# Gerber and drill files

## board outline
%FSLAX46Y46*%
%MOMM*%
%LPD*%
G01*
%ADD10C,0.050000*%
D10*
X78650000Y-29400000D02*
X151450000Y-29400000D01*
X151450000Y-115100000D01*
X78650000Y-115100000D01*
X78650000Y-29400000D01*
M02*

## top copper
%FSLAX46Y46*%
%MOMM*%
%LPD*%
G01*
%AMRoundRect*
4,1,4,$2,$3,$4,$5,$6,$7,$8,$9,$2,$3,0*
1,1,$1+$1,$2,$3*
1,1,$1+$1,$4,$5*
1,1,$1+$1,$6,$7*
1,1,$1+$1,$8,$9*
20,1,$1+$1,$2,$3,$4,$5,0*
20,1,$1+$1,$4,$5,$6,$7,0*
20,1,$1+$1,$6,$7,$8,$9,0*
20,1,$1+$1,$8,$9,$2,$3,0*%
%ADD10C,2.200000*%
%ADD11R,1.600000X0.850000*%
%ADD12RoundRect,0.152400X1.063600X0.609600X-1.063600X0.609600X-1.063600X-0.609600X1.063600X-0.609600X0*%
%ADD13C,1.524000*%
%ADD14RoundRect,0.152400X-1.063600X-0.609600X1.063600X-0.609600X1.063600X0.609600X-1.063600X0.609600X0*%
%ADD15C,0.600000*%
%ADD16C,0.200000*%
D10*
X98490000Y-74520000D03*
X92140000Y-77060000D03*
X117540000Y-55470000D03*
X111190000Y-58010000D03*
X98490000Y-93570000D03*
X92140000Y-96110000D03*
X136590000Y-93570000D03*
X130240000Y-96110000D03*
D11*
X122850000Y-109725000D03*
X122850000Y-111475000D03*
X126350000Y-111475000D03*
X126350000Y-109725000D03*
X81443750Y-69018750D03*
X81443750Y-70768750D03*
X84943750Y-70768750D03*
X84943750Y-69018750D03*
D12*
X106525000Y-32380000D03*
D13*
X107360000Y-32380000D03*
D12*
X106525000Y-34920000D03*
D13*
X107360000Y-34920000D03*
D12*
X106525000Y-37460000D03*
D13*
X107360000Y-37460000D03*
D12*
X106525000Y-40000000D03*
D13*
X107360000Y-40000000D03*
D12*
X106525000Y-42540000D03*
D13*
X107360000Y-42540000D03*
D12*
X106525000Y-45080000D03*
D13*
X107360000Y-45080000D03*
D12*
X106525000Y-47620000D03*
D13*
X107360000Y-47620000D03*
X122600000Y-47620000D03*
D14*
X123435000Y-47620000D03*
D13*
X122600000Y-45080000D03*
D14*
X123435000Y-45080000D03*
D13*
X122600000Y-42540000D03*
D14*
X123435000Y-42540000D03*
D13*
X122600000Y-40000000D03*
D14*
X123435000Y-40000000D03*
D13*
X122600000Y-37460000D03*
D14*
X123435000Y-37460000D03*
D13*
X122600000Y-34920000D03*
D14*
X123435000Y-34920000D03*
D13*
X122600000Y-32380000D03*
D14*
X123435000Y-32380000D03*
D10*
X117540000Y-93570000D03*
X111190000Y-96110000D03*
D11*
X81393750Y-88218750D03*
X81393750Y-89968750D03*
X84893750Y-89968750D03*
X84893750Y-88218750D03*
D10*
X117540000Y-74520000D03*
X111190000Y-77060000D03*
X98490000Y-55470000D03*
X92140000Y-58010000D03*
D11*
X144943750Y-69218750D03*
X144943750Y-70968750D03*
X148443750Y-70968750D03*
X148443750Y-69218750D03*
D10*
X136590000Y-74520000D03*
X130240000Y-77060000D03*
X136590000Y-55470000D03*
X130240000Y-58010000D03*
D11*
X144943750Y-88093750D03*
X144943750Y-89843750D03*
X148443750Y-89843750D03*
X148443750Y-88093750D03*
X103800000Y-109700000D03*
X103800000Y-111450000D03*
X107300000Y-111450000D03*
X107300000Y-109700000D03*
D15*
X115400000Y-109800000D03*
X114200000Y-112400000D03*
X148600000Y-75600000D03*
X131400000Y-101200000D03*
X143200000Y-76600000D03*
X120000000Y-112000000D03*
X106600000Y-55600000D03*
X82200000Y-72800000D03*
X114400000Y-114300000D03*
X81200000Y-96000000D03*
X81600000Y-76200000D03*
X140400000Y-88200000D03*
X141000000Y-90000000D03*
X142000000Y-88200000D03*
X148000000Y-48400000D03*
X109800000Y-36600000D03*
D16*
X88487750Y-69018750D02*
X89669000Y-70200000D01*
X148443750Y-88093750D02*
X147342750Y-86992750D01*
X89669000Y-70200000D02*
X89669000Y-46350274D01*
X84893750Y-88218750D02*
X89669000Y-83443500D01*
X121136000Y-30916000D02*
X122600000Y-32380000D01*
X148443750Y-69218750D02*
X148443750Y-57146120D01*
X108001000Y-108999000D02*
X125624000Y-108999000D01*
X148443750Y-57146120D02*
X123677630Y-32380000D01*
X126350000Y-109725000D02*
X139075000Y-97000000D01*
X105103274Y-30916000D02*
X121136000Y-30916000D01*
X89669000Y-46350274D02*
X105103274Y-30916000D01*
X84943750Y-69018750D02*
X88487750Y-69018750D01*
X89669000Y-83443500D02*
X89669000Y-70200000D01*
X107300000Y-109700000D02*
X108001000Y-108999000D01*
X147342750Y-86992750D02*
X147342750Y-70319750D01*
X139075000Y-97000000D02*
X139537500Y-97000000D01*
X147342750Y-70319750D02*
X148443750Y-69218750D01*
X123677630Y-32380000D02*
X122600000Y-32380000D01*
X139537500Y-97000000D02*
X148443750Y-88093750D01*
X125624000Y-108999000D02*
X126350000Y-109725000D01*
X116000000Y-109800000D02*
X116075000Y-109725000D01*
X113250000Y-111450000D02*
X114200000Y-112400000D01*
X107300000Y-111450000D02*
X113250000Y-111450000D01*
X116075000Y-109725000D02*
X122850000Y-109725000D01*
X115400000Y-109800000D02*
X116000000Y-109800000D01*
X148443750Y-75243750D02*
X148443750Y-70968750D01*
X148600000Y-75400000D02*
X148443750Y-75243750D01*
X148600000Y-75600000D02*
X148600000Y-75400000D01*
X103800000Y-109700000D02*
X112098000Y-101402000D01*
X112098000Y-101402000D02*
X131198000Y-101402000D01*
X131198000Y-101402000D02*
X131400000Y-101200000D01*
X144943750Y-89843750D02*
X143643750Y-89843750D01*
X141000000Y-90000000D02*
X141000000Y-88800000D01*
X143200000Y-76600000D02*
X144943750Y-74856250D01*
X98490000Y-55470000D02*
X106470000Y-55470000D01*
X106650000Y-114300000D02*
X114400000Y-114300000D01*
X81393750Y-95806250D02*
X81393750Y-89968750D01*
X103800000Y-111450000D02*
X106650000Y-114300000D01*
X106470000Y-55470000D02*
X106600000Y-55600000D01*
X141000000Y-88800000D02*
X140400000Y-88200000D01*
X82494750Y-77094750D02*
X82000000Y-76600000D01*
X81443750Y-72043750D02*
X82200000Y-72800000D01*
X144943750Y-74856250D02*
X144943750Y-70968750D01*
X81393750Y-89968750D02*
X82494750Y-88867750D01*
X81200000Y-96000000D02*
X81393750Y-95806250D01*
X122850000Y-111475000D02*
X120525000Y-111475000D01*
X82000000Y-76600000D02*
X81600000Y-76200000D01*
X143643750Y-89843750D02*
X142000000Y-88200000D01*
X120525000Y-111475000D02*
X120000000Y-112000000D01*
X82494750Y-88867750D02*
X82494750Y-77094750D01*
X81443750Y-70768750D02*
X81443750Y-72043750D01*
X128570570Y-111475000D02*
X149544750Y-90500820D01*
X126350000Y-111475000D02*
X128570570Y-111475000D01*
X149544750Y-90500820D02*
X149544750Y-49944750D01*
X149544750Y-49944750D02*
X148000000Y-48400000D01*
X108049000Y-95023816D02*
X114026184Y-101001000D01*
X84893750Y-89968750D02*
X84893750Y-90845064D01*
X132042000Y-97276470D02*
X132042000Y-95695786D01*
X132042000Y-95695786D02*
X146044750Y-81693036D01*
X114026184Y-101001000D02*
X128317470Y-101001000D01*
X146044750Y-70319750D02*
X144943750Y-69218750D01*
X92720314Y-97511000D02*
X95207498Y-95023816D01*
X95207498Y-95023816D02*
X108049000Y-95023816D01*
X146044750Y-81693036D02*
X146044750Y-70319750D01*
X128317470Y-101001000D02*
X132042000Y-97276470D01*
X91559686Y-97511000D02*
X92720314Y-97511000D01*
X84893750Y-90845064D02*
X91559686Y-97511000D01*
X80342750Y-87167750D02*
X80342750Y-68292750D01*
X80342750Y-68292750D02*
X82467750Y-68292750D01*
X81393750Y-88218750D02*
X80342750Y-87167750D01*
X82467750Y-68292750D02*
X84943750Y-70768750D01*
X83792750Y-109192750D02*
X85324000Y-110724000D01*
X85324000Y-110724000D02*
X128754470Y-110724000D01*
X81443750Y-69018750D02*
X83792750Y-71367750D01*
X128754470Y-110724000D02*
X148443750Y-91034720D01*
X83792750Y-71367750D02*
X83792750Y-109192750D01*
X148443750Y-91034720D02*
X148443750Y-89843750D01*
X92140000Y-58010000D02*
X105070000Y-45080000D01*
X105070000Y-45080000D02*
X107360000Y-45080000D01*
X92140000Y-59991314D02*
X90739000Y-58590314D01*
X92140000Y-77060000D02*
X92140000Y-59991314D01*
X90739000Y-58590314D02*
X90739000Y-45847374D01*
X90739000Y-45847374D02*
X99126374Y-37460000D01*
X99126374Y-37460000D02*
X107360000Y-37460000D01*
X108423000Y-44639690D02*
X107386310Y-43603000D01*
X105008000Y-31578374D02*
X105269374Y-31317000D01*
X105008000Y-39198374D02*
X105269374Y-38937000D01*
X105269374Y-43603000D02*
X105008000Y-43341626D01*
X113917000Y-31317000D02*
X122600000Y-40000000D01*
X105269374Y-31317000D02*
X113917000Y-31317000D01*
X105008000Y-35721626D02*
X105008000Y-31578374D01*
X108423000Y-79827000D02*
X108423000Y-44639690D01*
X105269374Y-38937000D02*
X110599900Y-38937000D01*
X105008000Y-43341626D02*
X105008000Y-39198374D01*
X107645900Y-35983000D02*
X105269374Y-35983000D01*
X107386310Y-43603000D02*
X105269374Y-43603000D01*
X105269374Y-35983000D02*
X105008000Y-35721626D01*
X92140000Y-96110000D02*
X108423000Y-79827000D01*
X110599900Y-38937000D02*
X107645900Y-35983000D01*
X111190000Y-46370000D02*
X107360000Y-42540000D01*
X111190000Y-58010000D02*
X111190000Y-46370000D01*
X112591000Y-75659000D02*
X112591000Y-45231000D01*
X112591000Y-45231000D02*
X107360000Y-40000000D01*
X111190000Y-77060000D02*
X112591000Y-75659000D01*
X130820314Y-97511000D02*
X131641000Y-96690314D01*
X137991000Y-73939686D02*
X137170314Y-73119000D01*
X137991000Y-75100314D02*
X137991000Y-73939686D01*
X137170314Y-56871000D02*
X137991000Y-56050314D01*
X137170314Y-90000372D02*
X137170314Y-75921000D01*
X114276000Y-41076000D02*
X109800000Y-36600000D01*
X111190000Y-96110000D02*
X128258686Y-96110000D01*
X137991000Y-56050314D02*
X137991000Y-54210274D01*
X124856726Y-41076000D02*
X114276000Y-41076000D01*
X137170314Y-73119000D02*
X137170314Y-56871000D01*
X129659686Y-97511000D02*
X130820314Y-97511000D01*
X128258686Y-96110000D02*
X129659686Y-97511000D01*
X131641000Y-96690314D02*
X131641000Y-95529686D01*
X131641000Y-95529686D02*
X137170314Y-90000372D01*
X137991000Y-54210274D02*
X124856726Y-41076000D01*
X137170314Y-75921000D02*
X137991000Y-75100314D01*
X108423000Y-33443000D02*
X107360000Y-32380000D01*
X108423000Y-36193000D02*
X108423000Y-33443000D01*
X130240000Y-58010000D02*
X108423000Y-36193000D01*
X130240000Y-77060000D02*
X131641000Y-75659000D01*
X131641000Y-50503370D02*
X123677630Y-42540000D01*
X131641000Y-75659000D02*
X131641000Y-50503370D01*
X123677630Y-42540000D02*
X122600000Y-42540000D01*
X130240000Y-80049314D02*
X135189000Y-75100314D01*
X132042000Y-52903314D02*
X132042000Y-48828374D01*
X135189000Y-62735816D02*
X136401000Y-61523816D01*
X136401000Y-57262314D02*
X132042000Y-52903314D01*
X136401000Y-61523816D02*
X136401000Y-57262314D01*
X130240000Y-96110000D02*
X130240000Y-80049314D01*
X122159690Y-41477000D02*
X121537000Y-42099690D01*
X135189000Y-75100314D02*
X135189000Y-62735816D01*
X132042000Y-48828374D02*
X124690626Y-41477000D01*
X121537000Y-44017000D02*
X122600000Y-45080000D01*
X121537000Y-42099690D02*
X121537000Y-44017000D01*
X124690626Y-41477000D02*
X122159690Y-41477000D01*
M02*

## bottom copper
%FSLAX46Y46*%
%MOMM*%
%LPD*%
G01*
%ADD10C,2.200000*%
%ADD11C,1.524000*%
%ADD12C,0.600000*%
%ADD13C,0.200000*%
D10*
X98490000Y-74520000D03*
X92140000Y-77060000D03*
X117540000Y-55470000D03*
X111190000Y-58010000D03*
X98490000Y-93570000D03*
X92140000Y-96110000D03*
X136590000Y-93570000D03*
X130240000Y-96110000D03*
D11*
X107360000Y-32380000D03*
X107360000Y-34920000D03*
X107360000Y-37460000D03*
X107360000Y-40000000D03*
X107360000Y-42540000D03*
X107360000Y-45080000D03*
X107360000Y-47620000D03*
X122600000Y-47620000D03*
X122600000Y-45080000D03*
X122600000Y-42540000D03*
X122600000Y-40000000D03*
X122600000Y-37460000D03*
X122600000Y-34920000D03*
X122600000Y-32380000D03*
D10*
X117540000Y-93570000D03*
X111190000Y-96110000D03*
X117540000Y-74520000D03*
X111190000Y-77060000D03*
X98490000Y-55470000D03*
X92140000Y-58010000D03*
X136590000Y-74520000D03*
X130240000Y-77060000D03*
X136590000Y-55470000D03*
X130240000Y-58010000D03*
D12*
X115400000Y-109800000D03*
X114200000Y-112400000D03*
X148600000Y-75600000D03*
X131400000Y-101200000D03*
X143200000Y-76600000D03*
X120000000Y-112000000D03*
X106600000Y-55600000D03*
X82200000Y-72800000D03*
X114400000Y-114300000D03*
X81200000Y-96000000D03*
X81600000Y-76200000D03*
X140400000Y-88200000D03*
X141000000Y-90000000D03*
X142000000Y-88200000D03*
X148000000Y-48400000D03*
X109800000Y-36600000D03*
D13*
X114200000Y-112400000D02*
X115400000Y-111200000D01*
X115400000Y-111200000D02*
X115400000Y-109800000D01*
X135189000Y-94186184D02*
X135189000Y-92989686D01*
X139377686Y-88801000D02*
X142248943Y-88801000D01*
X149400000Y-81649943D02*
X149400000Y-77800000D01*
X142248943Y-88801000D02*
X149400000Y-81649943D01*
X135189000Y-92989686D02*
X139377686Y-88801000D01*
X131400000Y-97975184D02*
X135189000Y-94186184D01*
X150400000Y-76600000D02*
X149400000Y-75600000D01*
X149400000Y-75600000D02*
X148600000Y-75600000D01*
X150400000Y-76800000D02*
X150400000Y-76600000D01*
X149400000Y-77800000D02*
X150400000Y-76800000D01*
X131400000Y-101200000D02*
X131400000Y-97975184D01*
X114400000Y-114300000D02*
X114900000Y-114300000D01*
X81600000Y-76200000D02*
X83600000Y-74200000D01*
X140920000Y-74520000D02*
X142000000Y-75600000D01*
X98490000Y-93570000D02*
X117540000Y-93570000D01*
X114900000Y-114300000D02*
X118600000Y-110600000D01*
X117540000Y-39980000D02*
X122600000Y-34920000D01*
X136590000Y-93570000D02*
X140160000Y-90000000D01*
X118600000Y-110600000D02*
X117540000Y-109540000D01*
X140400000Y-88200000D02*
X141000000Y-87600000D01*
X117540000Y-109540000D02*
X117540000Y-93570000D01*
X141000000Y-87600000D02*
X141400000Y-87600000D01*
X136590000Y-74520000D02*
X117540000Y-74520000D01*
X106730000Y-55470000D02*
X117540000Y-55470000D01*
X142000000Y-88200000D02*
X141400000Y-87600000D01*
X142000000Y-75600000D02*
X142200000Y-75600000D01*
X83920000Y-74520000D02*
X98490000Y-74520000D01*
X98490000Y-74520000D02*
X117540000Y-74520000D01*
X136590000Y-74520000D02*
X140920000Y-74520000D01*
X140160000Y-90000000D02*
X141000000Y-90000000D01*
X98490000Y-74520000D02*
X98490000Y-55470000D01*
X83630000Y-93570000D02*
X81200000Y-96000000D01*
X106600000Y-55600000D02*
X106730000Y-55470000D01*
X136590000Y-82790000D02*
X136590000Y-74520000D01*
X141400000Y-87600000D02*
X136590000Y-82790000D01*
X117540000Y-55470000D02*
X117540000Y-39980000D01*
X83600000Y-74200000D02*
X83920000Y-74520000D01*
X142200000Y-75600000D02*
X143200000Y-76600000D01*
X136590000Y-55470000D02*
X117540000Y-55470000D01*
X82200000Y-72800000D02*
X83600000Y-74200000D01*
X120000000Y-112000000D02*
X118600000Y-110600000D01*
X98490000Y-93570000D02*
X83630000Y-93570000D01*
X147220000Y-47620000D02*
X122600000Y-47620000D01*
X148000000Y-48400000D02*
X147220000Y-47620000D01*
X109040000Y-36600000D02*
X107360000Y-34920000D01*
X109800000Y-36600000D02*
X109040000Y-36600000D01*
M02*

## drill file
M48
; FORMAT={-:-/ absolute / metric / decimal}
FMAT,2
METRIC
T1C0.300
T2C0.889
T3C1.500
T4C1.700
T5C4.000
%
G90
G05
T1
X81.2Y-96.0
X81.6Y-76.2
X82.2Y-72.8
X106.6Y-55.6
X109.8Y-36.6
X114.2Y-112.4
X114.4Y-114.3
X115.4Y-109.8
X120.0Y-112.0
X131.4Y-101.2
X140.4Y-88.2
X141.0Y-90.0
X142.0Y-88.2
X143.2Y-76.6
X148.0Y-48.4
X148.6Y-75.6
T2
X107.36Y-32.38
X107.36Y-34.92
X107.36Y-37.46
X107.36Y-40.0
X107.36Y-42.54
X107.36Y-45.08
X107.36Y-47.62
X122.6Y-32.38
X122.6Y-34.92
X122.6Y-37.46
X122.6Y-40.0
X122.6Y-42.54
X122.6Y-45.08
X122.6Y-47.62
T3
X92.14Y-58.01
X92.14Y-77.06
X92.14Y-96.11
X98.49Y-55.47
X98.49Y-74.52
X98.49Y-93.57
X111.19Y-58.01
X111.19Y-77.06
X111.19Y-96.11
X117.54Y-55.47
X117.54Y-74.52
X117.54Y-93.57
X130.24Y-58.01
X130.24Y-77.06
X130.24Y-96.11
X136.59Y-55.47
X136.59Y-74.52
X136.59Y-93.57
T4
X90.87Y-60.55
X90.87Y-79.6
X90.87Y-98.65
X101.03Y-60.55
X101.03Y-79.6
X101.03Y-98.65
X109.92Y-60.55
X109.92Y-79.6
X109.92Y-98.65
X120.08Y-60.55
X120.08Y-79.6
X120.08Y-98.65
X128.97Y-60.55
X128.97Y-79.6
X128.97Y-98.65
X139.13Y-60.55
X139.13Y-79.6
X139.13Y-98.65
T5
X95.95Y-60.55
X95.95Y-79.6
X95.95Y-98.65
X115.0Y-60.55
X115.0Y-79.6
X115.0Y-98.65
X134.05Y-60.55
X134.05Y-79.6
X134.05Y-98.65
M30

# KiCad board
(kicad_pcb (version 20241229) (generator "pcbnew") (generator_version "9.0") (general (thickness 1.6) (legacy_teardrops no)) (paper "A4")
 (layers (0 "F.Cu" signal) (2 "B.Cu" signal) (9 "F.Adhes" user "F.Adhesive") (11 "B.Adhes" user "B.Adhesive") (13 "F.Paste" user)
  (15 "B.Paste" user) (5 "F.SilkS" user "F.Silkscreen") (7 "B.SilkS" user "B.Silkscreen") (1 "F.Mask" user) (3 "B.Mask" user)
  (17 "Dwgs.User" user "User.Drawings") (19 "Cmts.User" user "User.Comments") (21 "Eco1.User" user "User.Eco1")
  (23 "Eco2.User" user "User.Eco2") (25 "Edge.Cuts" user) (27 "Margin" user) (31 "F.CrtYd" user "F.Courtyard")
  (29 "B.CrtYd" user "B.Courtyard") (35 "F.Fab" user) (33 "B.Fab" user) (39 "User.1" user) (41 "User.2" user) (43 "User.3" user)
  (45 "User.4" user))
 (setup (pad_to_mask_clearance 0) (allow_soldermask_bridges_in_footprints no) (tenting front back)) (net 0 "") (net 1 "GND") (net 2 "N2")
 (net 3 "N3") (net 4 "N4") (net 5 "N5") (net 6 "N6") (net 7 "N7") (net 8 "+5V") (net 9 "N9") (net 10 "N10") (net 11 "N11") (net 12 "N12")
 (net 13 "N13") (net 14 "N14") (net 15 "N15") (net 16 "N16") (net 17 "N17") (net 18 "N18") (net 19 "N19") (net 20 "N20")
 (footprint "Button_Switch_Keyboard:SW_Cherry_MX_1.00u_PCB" (layer "F.Cu") (at 98.49 74.52)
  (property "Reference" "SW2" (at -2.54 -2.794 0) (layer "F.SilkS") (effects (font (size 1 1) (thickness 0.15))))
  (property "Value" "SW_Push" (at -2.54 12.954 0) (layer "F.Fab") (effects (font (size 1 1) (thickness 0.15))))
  (pad "" np_thru_hole circle (at -7.62 5.08) (size 1.7 1.7) (drill 1.7) (layers "*.Cu" "*.Mask"))
  (pad "" np_thru_hole circle (at -2.54 5.08) (size 4 4) (drill 4) (layers "*.Cu" "*.Mask"))
  (pad "" np_thru_hole circle (at 2.54 5.08) (size 1.7 1.7) (drill 1.7) (layers "*.Cu" "*.Mask"))
  (pad "1" thru_hole circle (at 0 0) (size 2.2 2.2) (drill 1.5) (layers "*.Cu" "*.Mask") (remove_unused_layers no) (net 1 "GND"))
  (pad "2" thru_hole circle (at -6.35 2.54) (size 2.2 2.2) (drill 1.5) (layers "*.Cu" "*.Mask") (remove_unused_layers no) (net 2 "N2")))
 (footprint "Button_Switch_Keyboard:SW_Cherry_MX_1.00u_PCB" (layer "F.Cu") (at 117.54 55.47)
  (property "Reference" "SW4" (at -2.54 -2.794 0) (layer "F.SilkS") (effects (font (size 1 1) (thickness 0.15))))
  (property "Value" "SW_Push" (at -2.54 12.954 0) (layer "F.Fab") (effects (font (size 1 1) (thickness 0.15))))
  (pad "" np_thru_hole circle (at -7.62 5.08) (size 1.7 1.7) (drill 1.7) (layers "*.Cu" "*.Mask"))
  (pad "" np_thru_hole circle (at -2.54 5.08) (size 4 4) (drill 4) (layers "*.Cu" "*.Mask"))
  (pad "" np_thru_hole circle (at 2.54 5.08) (size 1.7 1.7) (drill 1.7) (layers "*.Cu" "*.Mask"))
  (pad "1" thru_hole circle (at 0 0) (size 2.2 2.2) (drill 1.5) (layers "*.Cu" "*.Mask") (remove_unused_layers no) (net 1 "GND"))
  (pad "2" thru_hole circle (at -6.35 2.54) (size 2.2 2.2) (drill 1.5) (layers "*.Cu" "*.Mask") (remove_unused_layers no) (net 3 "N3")))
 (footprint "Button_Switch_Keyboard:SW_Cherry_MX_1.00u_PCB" (layer "F.Cu") (at 98.49 93.57)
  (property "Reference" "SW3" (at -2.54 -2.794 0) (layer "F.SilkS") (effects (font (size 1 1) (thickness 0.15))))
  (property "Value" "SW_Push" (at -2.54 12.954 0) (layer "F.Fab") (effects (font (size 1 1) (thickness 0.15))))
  (pad "" np_thru_hole circle (at -7.62 5.08) (size 1.7 1.7) (drill 1.7) (layers "*.Cu" "*.Mask"))
  (pad "" np_thru_hole circle (at -2.54 5.08) (size 4 4) (drill 4) (layers "*.Cu" "*.Mask"))
  (pad "" np_thru_hole circle (at 2.54 5.08) (size 1.7 1.7) (drill 1.7) (layers "*.Cu" "*.Mask"))
  (pad "1" thru_hole circle (at 0 0) (size 2.2 2.2) (drill 1.5) (layers "*.Cu" "*.Mask") (remove_unused_layers no) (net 1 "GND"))
  (pad "2" thru_hole circle (at -6.35 2.54) (size 2.2 2.2) (drill 1.5) (layers "*.Cu" "*.Mask") (remove_unused_layers no) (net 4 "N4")))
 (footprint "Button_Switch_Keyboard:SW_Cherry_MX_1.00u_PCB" (layer "F.Cu") (at 136.59 93.57)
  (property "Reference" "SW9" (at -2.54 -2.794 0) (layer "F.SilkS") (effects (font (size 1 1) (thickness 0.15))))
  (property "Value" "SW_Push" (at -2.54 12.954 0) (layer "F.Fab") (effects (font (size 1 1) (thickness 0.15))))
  (pad "" np_thru_hole circle (at -7.62 5.08) (size 1.7 1.7) (drill 1.7) (layers "*.Cu" "*.Mask"))
  (pad "" np_thru_hole circle (at -2.54 5.08) (size 4 4) (drill 4) (layers "*.Cu" "*.Mask"))
  (pad "" np_thru_hole circle (at 2.54 5.08) (size 1.7 1.7) (drill 1.7) (layers "*.Cu" "*.Mask"))
  (pad "1" thru_hole circle (at 0 0) (size 2.2 2.2) (drill 1.5) (layers "*.Cu" "*.Mask") (remove_unused_layers no) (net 1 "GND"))
  (pad "2" thru_hole circle (at -6.35 2.54) (size 2.2 2.2) (drill 1.5) (layers "*.Cu" "*.Mask") (remove_unused_layers no) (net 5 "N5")))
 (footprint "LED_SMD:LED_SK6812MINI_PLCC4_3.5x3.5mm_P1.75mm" (layer "F.Cu") (at 124.6 110.6)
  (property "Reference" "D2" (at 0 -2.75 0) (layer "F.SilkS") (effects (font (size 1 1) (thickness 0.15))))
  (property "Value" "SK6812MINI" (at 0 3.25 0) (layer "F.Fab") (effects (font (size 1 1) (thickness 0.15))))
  (pad "1" smd rect (at -1.75 -0.875) (size 1.6 0.85) (layers "F.Cu" "F.Mask" "F.Paste") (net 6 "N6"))
  (pad "2" smd rect (at -1.75 0.875) (size 1.6 0.85) (layers "F.Cu" "F.Mask" "F.Paste") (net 1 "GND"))
  (pad "3" smd rect (at 1.75 0.875) (size 1.6 0.85) (layers "F.Cu" "F.Mask" "F.Paste") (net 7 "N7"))
  (pad "4" smd rect (at 1.75 -0.875) (size 1.6 0.85) (layers "F.Cu" "F.Mask" "F.Paste") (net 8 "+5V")))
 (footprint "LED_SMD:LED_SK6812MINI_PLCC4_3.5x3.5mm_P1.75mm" (layer "F.Cu") (at 83.19375 69.89375)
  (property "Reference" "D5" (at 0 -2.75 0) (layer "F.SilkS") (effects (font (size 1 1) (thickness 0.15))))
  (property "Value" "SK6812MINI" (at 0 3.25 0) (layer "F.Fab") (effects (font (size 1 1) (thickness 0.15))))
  (pad "1" smd rect (at -1.75 -0.875) (size 1.6 0.85) (layers "F.Cu" "F.Mask" "F.Paste") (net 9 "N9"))
  (pad "2" smd rect (at -1.75 0.875) (size 1.6 0.85) (layers "F.Cu" "F.Mask" "F.Paste") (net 1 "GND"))
  (pad "3" smd rect (at 1.75 0.875) (size 1.6 0.85) (layers "F.Cu" "F.Mask" "F.Paste") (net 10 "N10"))
  (pad "4" smd rect (at 1.75 -0.875) (size 1.6 0.85) (layers "F.Cu" "F.Mask" "F.Paste") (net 8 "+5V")))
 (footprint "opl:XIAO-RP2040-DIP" (layer "F.Cu") (at 114.98 40)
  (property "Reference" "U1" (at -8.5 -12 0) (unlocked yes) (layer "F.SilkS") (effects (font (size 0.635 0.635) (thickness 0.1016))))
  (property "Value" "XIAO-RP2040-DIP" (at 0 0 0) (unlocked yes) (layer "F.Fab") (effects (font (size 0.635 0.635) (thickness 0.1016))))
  (pad "1" smd roundrect (at -8.455 -7.62 180) (size 2.432 1.524) (layers "F.Cu" "F.Mask") (roundrect_rratio 0.1) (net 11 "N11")
   (thermal_bridge_angle 45))
  (pad "1" thru_hole circle (at -7.62 -7.62 180) (size 1.524 1.524) (drill 0.889) (layers "*.Cu" "*.Mask") (remove_unused_layers no)
   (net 11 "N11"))
  (pad "2" smd roundrect (at -8.455 -5.08 180) (size 2.432 1.524) (layers "F.Cu" "F.Mask") (roundrect_rratio 0.1) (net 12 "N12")
   (thermal_bridge_angle 45))
  (pad "2" thru_hole circle (at -7.62 -5.08 180) (size 1.524 1.524) (drill 0.889) (layers "*.Cu" "*.Mask") (remove_unused_layers no)
   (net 12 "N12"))
  (pad "3" smd roundrect (at -8.455 -2.54 180) (size 2.432 1.524) (layers "F.Cu" "F.Mask") (roundrect_rratio 0.1) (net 2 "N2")
   (thermal_bridge_angle 45))
  (pad "3" thru_hole circle (at -7.62 -2.54 180) (size 1.524 1.524) (drill 0.889) (layers "*.Cu" "*.Mask") (remove_unused_layers no)
   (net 2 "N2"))
  (pad "4" smd roundrect (at -8.455 0 180) (size 2.432 1.524) (layers "F.Cu" "F.Mask") (roundrect_rratio 0.1) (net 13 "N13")
   (thermal_bridge_angle 45))
  (pad "4" thru_hole circle (at -7.62 0 180) (size 1.524 1.524) (drill 0.889) (layers "*.Cu" "*.Mask") (remove_unused_layers no)
   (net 13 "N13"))
  (pad "5" smd roundrect (at -8.455 2.54 180) (size 2.432 1.524) (layers "F.Cu" "F.Mask") (roundrect_rratio 0.1) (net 3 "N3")
   (thermal_bridge_angle 45))
  (pad "5" thru_hole circle (at -7.62 2.54 180) (size 1.524 1.524) (drill 0.889) (layers "*.Cu" "*.Mask") (remove_unused_layers no)
   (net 3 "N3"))
  (pad "6" smd roundrect (at -8.455 5.08 180) (size 2.432 1.524) (layers "F.Cu" "F.Mask") (roundrect_rratio 0.1) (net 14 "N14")
   (thermal_bridge_angle 45))
  (pad "6" thru_hole circle (at -7.62 5.08 180) (size 1.524 1.524) (drill 0.889) (layers "*.Cu" "*.Mask") (remove_unused_layers no)
   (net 14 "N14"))
  (pad "7" smd roundrect (at -8.455 7.62 180) (size 2.432 1.524) (layers "F.Cu" "F.Mask") (roundrect_rratio 0.1) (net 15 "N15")
   (thermal_bridge_angle 45))
  (pad "7" thru_hole circle (at -7.62 7.62 180) (size 1.524 1.524) (drill 0.889) (layers "*.Cu" "*.Mask") (remove_unused_layers no)
   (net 15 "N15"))
  (pad "8" thru_hole circle (at 7.62 7.62) (size 1.524 1.524) (drill 0.889) (layers "*.Cu" "*.Mask") (remove_unused_layers no) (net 7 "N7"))
  (pad "8" smd roundrect (at 8.455 7.62) (size 2.432 1.524) (layers "F.Cu" "F.Mask") (roundrect_rratio 0.1) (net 7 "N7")
   (thermal_bridge_angle 45))
  (pad "9" thru_hole circle (at 7.62 5.08) (size 1.524 1.524) (drill 0.889) (layers "*.Cu" "*.Mask") (remove_unused_layers no) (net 5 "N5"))
  (pad "9" smd roundrect (at 8.455 5.08) (size 2.432 1.524) (layers "F.Cu" "F.Mask") (roundrect_rratio 0.1) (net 5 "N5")
   (thermal_bridge_angle 45))
  (pad "10" thru_hole circle (at 7.62 2.54) (size 1.524 1.524) (drill 0.889) (layers "*.Cu" "*.Mask") (remove_unused_layers no)
   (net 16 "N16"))
  (pad "10" smd roundrect (at 8.455 2.54) (size 2.432 1.524) (layers "F.Cu" "F.Mask") (roundrect_rratio 0.1) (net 16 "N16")
   (thermal_bridge_angle 45))
  (pad "11" thru_hole circle (at 7.62 0) (size 1.524 1.524) (drill 0.889) (layers "*.Cu" "*.Mask") (remove_unused_layers no) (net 4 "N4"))
  (pad "11" smd roundrect (at 8.455 0) (size 2.432 1.524) (layers "F.Cu" "F.Mask") (roundrect_rratio 0.1) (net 4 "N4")
   (thermal_bridge_angle 45))
  (pad "12" thru_hole circle (at 7.62 -2.54) (size 1.524 1.524) (drill 0.889) (layers "*.Cu" "*.Mask") (remove_unused_layers no)
   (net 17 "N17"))
  (pad "12" smd roundrect (at 8.455 -2.54) (size 2.432 1.524) (layers "F.Cu" "F.Mask") (roundrect_rratio 0.1) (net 17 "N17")
   (thermal_bridge_angle 45))
  (pad "13" thru_hole circle (at 7.62 -5.08) (size 1.524 1.524) (drill 0.889) (layers "*.Cu" "*.Mask") (remove_unused_layers no)
   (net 1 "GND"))
  (pad "13" smd roundrect (at 8.455 -5.08) (size 2.432 1.524) (layers "F.Cu" "F.Mask") (roundrect_rratio 0.1) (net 1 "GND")
   (thermal_bridge_angle 45))
  (pad "14" thru_hole circle (at 7.62 -7.62) (size 1.524 1.524) (drill 0.889) (layers "*.Cu" "*.Mask") (remove_unused_layers no)
   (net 8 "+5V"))
  (pad "14" smd roundrect (at 8.455 -7.62) (size 2.432 1.524) (layers "F.Cu" "F.Mask") (roundrect_rratio 0.1) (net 8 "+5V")
   (thermal_bridge_angle 45)))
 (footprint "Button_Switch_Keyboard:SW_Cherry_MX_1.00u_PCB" (layer "F.Cu") (at 117.54 93.57)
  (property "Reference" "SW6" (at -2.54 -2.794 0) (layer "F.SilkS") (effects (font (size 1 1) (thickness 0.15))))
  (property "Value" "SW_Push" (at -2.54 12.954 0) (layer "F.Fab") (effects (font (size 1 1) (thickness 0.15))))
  (pad "" np_thru_hole circle (at -7.62 5.08) (size 1.7 1.7) (drill 1.7) (layers "*.Cu" "*.Mask"))
  (pad "" np_thru_hole circle (at -2.54 5.08) (size 4 4) (drill 4) (layers "*.Cu" "*.Mask"))
  (pad "" np_thru_hole circle (at 2.54 5.08) (size 1.7 1.7) (drill 1.7) (layers "*.Cu" "*.Mask"))
  (pad "1" thru_hole circle (at 0 0) (size 2.2 2.2) (drill 1.5) (layers "*.Cu" "*.Mask") (remove_unused_layers no) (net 1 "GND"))
  (pad "2" thru_hole circle (at -6.35 2.54) (size 2.2 2.2) (drill 1.5) (layers "*.Cu" "*.Mask") (remove_unused_layers no) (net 12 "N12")))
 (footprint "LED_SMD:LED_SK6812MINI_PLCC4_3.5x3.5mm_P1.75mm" (layer "F.Cu") (at 83.14375 89.09375)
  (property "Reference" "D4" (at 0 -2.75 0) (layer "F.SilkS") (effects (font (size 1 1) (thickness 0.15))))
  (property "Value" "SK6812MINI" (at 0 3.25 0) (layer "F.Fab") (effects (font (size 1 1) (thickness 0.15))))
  (pad "1" smd rect (at -1.75 -0.875) (size 1.6 0.85) (layers "F.Cu" "F.Mask" "F.Paste") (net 10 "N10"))
  (pad "2" smd rect (at -1.75 0.875) (size 1.6 0.85) (layers "F.Cu" "F.Mask" "F.Paste") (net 1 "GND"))
  (pad "3" smd rect (at 1.75 0.875) (size 1.6 0.85) (layers "F.Cu" "F.Mask" "F.Paste") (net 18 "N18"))
  (pad "4" smd rect (at 1.75 -0.875) (size 1.6 0.85) (layers "F.Cu" "F.Mask" "F.Paste") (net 8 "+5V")))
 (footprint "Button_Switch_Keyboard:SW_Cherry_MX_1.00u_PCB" (layer "F.Cu") (at 117.54 74.52)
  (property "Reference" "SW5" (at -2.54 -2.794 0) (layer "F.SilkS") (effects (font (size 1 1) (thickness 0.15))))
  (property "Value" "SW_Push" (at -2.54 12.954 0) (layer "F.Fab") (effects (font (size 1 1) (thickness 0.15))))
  (pad "" np_thru_hole circle (at -7.62 5.08) (size 1.7 1.7) (drill 1.7) (layers "*.Cu" "*.Mask"))
  (pad "" np_thru_hole circle (at -2.54 5.08) (size 4 4) (drill 4) (layers "*.Cu" "*.Mask"))
  (pad "" np_thru_hole circle (at 2.54 5.08) (size 1.7 1.7) (drill 1.7) (layers "*.Cu" "*.Mask"))
  (pad "1" thru_hole circle (at 0 0) (size 2.2 2.2) (drill 1.5) (layers "*.Cu" "*.Mask") (remove_unused_layers no) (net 1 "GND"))
  (pad "2" thru_hole circle (at -6.35 2.54) (size 2.2 2.2) (drill 1.5) (layers "*.Cu" "*.Mask") (remove_unused_layers no) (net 13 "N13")))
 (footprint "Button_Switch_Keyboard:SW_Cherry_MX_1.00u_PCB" (layer "F.Cu") (at 98.49 55.47)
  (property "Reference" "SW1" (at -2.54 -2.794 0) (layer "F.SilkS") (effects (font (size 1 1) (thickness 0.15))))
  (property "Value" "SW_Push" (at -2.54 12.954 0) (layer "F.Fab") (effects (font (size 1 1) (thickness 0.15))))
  (pad "" np_thru_hole circle (at -7.62 5.08) (size 1.7 1.7) (drill 1.7) (layers "*.Cu" "*.Mask"))
  (pad "" np_thru_hole circle (at -2.54 5.08) (size 4 4) (drill 4) (layers "*.Cu" "*.Mask"))
  (pad "" np_thru_hole circle (at 2.54 5.08) (size 1.7 1.7) (drill 1.7) (layers "*.Cu" "*.Mask"))
  (pad "1" thru_hole circle (at 0 0) (size 2.2 2.2) (drill 1.5) (layers "*.Cu" "*.Mask") (remove_unused_layers no) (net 1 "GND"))
  (pad "2" thru_hole circle (at -6.35 2.54) (size 2.2 2.2) (drill 1.5) (layers "*.Cu" "*.Mask") (remove_unused_layers no) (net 14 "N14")))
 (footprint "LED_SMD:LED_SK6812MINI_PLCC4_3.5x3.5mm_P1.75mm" (layer "F.Cu") (at 146.69375 70.09375)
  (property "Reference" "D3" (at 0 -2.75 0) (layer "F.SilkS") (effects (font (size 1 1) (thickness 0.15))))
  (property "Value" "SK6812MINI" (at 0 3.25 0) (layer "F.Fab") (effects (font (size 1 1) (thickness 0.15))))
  (pad "1" smd rect (at -1.75 -0.875) (size 1.6 0.85) (layers "F.Cu" "F.Mask" "F.Paste") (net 18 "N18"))
  (pad "2" smd rect (at -1.75 0.875) (size 1.6 0.85) (layers "F.Cu" "F.Mask" "F.Paste") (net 1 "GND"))
  (pad "3" smd rect (at 1.75 0.875) (size 1.6 0.85) (layers "F.Cu" "F.Mask" "F.Paste") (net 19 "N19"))
  (pad "4" smd rect (at 1.75 -0.875) (size 1.6 0.85) (layers "F.Cu" "F.Mask" "F.Paste") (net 8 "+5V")))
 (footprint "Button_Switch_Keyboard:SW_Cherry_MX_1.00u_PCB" (layer "F.Cu") (at 136.59 74.52)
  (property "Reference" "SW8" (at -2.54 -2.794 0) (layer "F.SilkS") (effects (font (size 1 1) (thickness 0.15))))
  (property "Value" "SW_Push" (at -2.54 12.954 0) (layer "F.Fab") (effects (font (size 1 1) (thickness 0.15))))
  (pad "" np_thru_hole circle (at -7.62 5.08) (size 1.7 1.7) (drill 1.7) (layers "*.Cu" "*.Mask"))
  (pad "" np_thru_hole circle (at -2.54 5.08) (size 4 4) (drill 4) (layers "*.Cu" "*.Mask"))
  (pad "" np_thru_hole circle (at 2.54 5.08) (size 1.7 1.7) (drill 1.7) (layers "*.Cu" "*.Mask"))
  (pad "1" thru_hole circle (at 0 0) (size 2.2 2.2) (drill 1.5) (layers "*.Cu" "*.Mask") (remove_unused_layers no) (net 1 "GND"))
  (pad "2" thru_hole circle (at -6.35 2.54) (size 2.2 2.2) (drill 1.5) (layers "*.Cu" "*.Mask") (remove_unused_layers no) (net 16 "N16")))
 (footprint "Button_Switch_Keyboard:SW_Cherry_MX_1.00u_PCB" (layer "F.Cu") (at 136.59 55.47)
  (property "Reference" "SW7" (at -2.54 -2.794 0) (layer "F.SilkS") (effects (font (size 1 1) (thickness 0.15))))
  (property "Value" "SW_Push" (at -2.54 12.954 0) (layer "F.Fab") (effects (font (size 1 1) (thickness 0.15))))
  (pad "" np_thru_hole circle (at -7.62 5.08) (size 1.7 1.7) (drill 1.7) (layers "*.Cu" "*.Mask"))
  (pad "" np_thru_hole circle (at -2.54 5.08) (size 4 4) (drill 4) (layers "*.Cu" "*.Mask"))
  (pad "" np_thru_hole circle (at 2.54 5.08) (size 1.7 1.7) (drill 1.7) (layers "*.Cu" "*.Mask"))
  (pad "1" thru_hole circle (at 0 0) (size 2.2 2.2) (drill 1.5) (layers "*.Cu" "*.Mask") (remove_unused_layers no) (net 1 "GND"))
  (pad "2" thru_hole circle (at -6.35 2.54) (size 2.2 2.2) (drill 1.5) (layers "*.Cu" "*.Mask") (remove_unused_layers no) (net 11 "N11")))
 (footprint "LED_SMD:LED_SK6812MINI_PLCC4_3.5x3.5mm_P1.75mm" (layer "F.Cu") (at 146.69375 88.96875)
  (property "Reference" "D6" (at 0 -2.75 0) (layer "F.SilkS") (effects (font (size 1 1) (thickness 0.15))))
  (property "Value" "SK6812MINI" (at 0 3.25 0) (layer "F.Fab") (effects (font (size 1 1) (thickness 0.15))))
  (pad "1" smd rect (at -1.75 -0.875) (size 1.6 0.85) (layers "F.Cu" "F.Mask" "F.Paste") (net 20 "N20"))
  (pad "2" smd rect (at -1.75 0.875) (size 1.6 0.85) (layers "F.Cu" "F.Mask" "F.Paste") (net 1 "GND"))
  (pad "3" smd rect (at 1.75 0.875) (size 1.6 0.85) (layers "F.Cu" "F.Mask" "F.Paste") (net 9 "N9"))
  (pad "4" smd rect (at 1.75 -0.875) (size 1.6 0.85) (layers "F.Cu" "F.Mask" "F.Paste") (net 8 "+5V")))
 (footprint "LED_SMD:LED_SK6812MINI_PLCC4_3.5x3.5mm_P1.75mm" (layer "F.Cu") (at 105.55 110.575)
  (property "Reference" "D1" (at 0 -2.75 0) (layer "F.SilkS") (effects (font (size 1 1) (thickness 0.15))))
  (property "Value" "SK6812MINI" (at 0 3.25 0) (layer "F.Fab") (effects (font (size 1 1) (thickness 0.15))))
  (pad "1" smd rect (at -1.75 -0.875) (size 1.6 0.85) (layers "F.Cu" "F.Mask" "F.Paste") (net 19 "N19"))
  (pad "2" smd rect (at -1.75 0.875) (size 1.6 0.85) (layers "F.Cu" "F.Mask" "F.Paste") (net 1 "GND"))
  (pad "3" smd rect (at 1.75 0.875) (size 1.6 0.85) (layers "F.Cu" "F.Mask" "F.Paste") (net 6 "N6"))
  (pad "4" smd rect (at 1.75 -0.875) (size 1.6 0.85) (layers "F.Cu" "F.Mask" "F.Paste") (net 8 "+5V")))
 (gr_rect (start 78.65 29.4) (end 151.45 115.1) (stroke (width 0.05) (type default)) (fill no) (layer "Edge.Cuts"))
 (segment (start 88.48775 69.01875) (end 89.669 70.2) (width 0.2) (layer "F.Cu") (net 8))
 (segment (start 148.44375 88.09375) (end 147.34275 86.99275) (width 0.2) (layer "F.Cu") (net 8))
 (segment (start 89.669 70.2) (end 89.669 46.350274) (width 0.2) (layer "F.Cu") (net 8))
 (segment (start 84.89375 88.21875) (end 89.669 83.4435) (width 0.2) (layer "F.Cu") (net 8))
 (segment (start 121.136 30.916) (end 122.6 32.38) (width 0.2) (layer "F.Cu") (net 8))
 (segment (start 148.44375 69.21875) (end 148.44375 57.14612) (width 0.2) (layer "F.Cu") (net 8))
 (segment (start 108.001 108.999) (end 125.624 108.999) (width 0.2) (layer "F.Cu") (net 8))
 (segment (start 148.44375 57.14612) (end 123.67763 32.38) (width 0.2) (layer "F.Cu") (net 8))
 (segment (start 126.35 109.725) (end 139.075 97) (width 0.2) (layer "F.Cu") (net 8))
 (segment (start 105.103274 30.916) (end 121.136 30.916) (width 0.2) (layer "F.Cu") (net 8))
 (segment (start 89.669 46.350274) (end 105.103274 30.916) (width 0.2) (layer "F.Cu") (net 8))
 (segment (start 84.94375 69.01875) (end 88.48775 69.01875) (width 0.2) (layer "F.Cu") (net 8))
 (segment (start 89.669 83.4435) (end 89.669 70.2) (width 0.2) (layer "F.Cu") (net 8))
 (segment (start 107.3 109.7) (end 108.001 108.999) (width 0.2) (layer "F.Cu") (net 8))
 (segment (start 147.34275 86.99275) (end 147.34275 70.31975) (width 0.2) (layer "F.Cu") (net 8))
 (segment (start 139.075 97) (end 139.5375 97) (width 0.2) (layer "F.Cu") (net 8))
 (segment (start 147.34275 70.31975) (end 148.44375 69.21875) (width 0.2) (layer "F.Cu") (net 8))
 (segment (start 123.67763 32.38) (end 122.6 32.38) (width 0.2) (layer "F.Cu") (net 8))
 (segment (start 139.5375 97) (end 148.44375 88.09375) (width 0.2) (layer "F.Cu") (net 8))
 (segment (start 125.624 108.999) (end 126.35 109.725) (width 0.2) (layer "F.Cu") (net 8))
 (segment (start 116 109.8) (end 116.075 109.725) (width 0.2) (layer "F.Cu") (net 6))
 (segment (start 113.25 111.45) (end 114.2 112.4) (width 0.2) (layer "F.Cu") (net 6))
 (segment (start 107.3 111.45) (end 113.25 111.45) (width 0.2) (layer "F.Cu") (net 6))
 (segment (start 116.075 109.725) (end 122.85 109.725) (width 0.2) (layer "F.Cu") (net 6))
 (segment (start 115.4 109.8) (end 116 109.8) (width 0.2) (layer "F.Cu") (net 6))
 (via (at 115.4 109.8) (size 0.6) (drill 0.3) (layers "F.Cu" "B.Cu") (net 6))
 (via (at 114.2 112.4) (size 0.6) (drill 0.3) (layers "F.Cu" "B.Cu") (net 6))
 (segment (start 114.2 112.4) (end 115.4 111.2) (width 0.2) (layer "B.Cu") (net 6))
 (segment (start 115.4 111.2) (end 115.4 109.8) (width 0.2) (layer "B.Cu") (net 6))
 (segment (start 148.44375 75.24375) (end 148.44375 70.96875) (width 0.2) (layer "F.Cu") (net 19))
 (segment (start 148.6 75.4) (end 148.44375 75.24375) (width 0.2) (layer "F.Cu") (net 19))
 (segment (start 148.6 75.6) (end 148.6 75.4) (width 0.2) (layer "F.Cu") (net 19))
 (segment (start 103.8 109.7) (end 112.098 101.402) (width 0.2) (layer "F.Cu") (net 19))
 (segment (start 112.098 101.402) (end 131.198 101.402) (width 0.2) (layer "F.Cu") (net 19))
 (segment (start 131.198 101.402) (end 131.4 101.2) (width 0.2) (layer "F.Cu") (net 19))
 (via (at 148.6 75.6) (size 0.6) (drill 0.3) (layers "F.Cu" "B.Cu") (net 19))
 (via (at 131.4 101.2) (size 0.6) (drill 0.3) (layers "F.Cu" "B.Cu") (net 19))
 (segment (start 135.189 94.186184) (end 135.189 92.989686) (width 0.2) (layer "B.Cu") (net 19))
 (segment (start 139.377686 88.801) (end 142.248943 88.801) (width 0.2) (layer "B.Cu") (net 19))
 (segment (start 149.4 81.649943) (end 149.4 77.8) (width 0.2) (layer "B.Cu") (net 19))
 (segment (start 142.248943 88.801) (end 149.4 81.649943) (width 0.2) (layer "B.Cu") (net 19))
 (segment (start 135.189 92.989686) (end 139.377686 88.801) (width 0.2) (layer "B.Cu") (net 19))
 (segment (start 131.4 97.975184) (end 135.189 94.186184) (width 0.2) (layer "B.Cu") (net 19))
 (segment (start 150.4 76.6) (end 149.4 75.6) (width 0.2) (layer "B.Cu") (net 19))
 (segment (start 149.4 75.6) (end 148.6 75.6) (width 0.2) (layer "B.Cu") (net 19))
 (segment (start 150.4 76.8) (end 150.4 76.6) (width 0.2) (layer "B.Cu") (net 19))
 (segment (start 149.4 77.8) (end 150.4 76.8) (width 0.2) (layer "B.Cu") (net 19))
 (segment (start 131.4 101.2) (end 131.4 97.975184) (width 0.2) (layer "B.Cu") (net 19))
 (segment (start 144.94375 89.84375) (end 143.64375 89.84375) (width 0.2) (layer "F.Cu") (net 1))
 (segment (start 141 90) (end 141 88.8) (width 0.2) (layer "F.Cu") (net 1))
 (segment (start 143.2 76.6) (end 144.94375 74.85625) (width 0.2) (layer "F.Cu") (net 1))
 (segment (start 98.49 55.47) (end 106.47 55.47) (width 0.2) (layer "F.Cu") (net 1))
 (segment (start 106.65 114.3) (end 114.4 114.3) (width 0.2) (layer "F.Cu") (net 1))
 (segment (start 81.39375 95.80625) (end 81.39375 89.96875) (width 0.2) (layer "F.Cu") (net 1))
 (segment (start 103.8 111.45) (end 106.65 114.3) (width 0.2) (layer "F.Cu") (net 1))
 (segment (start 106.47 55.47) (end 106.6 55.6) (width 0.2) (layer "F.Cu") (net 1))
 (segment (start 141 88.8) (end 140.4 88.2) (width 0.2) (layer "F.Cu") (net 1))
 (segment (start 82.49475 77.09475) (end 82 76.6) (width 0.2) (layer "F.Cu") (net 1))
 (segment (start 81.44375 72.04375) (end 82.2 72.8) (width 0.2) (layer "F.Cu") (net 1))
 (segment (start 144.94375 74.85625) (end 144.94375 70.96875) (width 0.2) (layer "F.Cu") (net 1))
 (segment (start 81.39375 89.96875) (end 82.49475 88.86775) (width 0.2) (layer "F.Cu") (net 1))
 (segment (start 81.2 96) (end 81.39375 95.80625) (width 0.2) (layer "F.Cu") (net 1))
 (segment (start 122.85 111.475) (end 120.525 111.475) (width 0.2) (layer "F.Cu") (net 1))
 (segment (start 82 76.6) (end 81.6 76.2) (width 0.2) (layer "F.Cu") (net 1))
 (segment (start 143.64375 89.84375) (end 142 88.2) (width 0.2) (layer "F.Cu") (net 1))
 (segment (start 120.525 111.475) (end 120 112) (width 0.2) (layer "F.Cu") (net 1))
 (segment (start 82.49475 88.86775) (end 82.49475 77.09475) (width 0.2) (layer "F.Cu") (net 1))
 (segment (start 81.44375 70.76875) (end 81.44375 72.04375) (width 0.2) (layer "F.Cu") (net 1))
 (via (at 143.2 76.6) (size 0.6) (drill 0.3) (layers "F.Cu" "B.Cu") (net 1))
 (via (at 120 112) (size 0.6) (drill 0.3) (layers "F.Cu" "B.Cu") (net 1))
 (via (at 106.6 55.6) (size 0.6) (drill 0.3) (layers "F.Cu" "B.Cu") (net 1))
 (via (at 82.2 72.8) (size 0.6) (drill 0.3) (layers "F.Cu" "B.Cu") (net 1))
 (via (at 114.4 114.3) (size 0.6) (drill 0.3) (layers "F.Cu" "B.Cu") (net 1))
 (via (at 81.2 96) (size 0.6) (drill 0.3) (layers "F.Cu" "B.Cu") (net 1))
 (via (at 81.6 76.2) (size 0.6) (drill 0.3) (layers "F.Cu" "B.Cu") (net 1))
 (via (at 140.4 88.2) (size 0.6) (drill 0.3) (layers "F.Cu" "B.Cu") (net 1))
 (via (at 141 90) (size 0.6) (drill 0.3) (layers "F.Cu" "B.Cu") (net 1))
 (via (at 142 88.2) (size 0.6) (drill 0.3) (layers "F.Cu" "B.Cu") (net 1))
 (segment (start 114.4 114.3) (end 114.9 114.3) (width 0.2) (layer "B.Cu") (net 1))
 (segment (start 81.6 76.2) (end 83.6 74.2) (width 0.2) (layer "B.Cu") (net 1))
 (segment (start 140.92 74.52) (end 142 75.6) (width 0.2) (layer "B.Cu") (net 1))
 (segment (start 98.49 93.57) (end 117.54 93.57) (width 0.2) (layer "B.Cu") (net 1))
 (segment (start 114.9 114.3) (end 118.6 110.6) (width 0.2) (layer "B.Cu") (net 1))
 (segment (start 117.54 39.98) (end 122.6 34.92) (width 0.2) (layer "B.Cu") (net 1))
 (segment (start 136.59 93.57) (end 140.16 90) (width 0.2) (layer "B.Cu") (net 1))
 (segment (start 118.6 110.6) (end 117.54 109.54) (width 0.2) (layer "B.Cu") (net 1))
 (segment (start 140.4 88.2) (end 141 87.6) (width 0.2) (layer "B.Cu") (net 1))
 (segment (start 117.54 109.54) (end 117.54 93.57) (width 0.2) (layer "B.Cu") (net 1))
 (segment (start 141 87.6) (end 141.4 87.6) (width 0.2) (layer "B.Cu") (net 1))
 (segment (start 136.59 74.52) (end 117.54 74.52) (width 0.2) (layer "B.Cu") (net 1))
 (segment (start 106.73 55.47) (end 117.54 55.47) (width 0.2) (layer "B.Cu") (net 1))
 (segment (start 142 88.2) (end 141.4 87.6) (width 0.2) (layer "B.Cu") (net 1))
 (segment (start 142 75.6) (end 142.2 75.6) (width 0.2) (layer "B.Cu") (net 1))
 (segment (start 83.92 74.52) (end 98.49 74.52) (width 0.2) (layer "B.Cu") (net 1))
 (segment (start 98.49 74.52) (end 117.54 74.52) (width 0.2) (layer "B.Cu") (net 1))
 (segment (start 136.59 74.52) (end 140.92 74.52) (width 0.2) (layer "B.Cu") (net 1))
 (segment (start 140.16 90) (end 141 90) (width 0.2) (layer "B.Cu") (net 1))
 (segment (start 98.49 74.52) (end 98.49 55.47) (width 0.2) (layer "B.Cu") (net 1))
 (segment (start 83.63 93.57) (end 81.2 96) (width 0.2) (layer "B.Cu") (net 1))
 (segment (start 106.6 55.6) (end 106.73 55.47) (width 0.2) (layer "B.Cu") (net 1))
 (segment (start 136.59 82.79) (end 136.59 74.52) (width 0.2) (layer "B.Cu") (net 1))
 (segment (start 141.4 87.6) (end 136.59 82.79) (width 0.2) (layer "B.Cu") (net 1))
 (segment (start 117.54 55.47) (end 117.54 39.98) (width 0.2) (layer "B.Cu") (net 1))
 (segment (start 83.6 74.2) (end 83.92 74.52) (width 0.2) (layer "B.Cu") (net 1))
 (segment (start 142.2 75.6) (end 143.2 76.6) (width 0.2) (layer "B.Cu") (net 1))
 (segment (start 136.59 55.47) (end 117.54 55.47) (width 0.2) (layer "B.Cu") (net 1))
 (segment (start 82.2 72.8) (end 83.6 74.2) (width 0.2) (layer "B.Cu") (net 1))
 (segment (start 120 112) (end 118.6 110.6) (width 0.2) (layer "B.Cu") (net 1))
 (segment (start 98.49 93.57) (end 83.63 93.57) (width 0.2) (layer "B.Cu") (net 1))
 (segment (start 128.57057 111.475) (end 149.54475 90.50082) (width 0.2) (layer "F.Cu") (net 7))
 (segment (start 126.35 111.475) (end 128.57057 111.475) (width 0.2) (layer "F.Cu") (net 7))
 (segment (start 149.54475 90.50082) (end 149.54475 49.94475) (width 0.2) (layer "F.Cu") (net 7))
 (segment (start 149.54475 49.94475) (end 148 48.4) (width 0.2) (layer "F.Cu") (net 7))
 (via (at 148 48.4) (size 0.6) (drill 0.3) (layers "F.Cu" "B.Cu") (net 7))
 (segment (start 147.22 47.62) (end 122.6 47.62) (width 0.2) (layer "B.Cu") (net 7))
 (segment (start 148 48.4) (end 147.22 47.62) (width 0.2) (layer "B.Cu") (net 7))
 (segment (start 108.049 95.023816) (end 114.026184 101.001) (width 0.2) (layer "F.Cu") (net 18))
 (segment (start 84.89375 89.96875) (end 84.89375 90.845064) (width 0.2) (layer "F.Cu") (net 18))
 (segment (start 132.042 97.27647) (end 132.042 95.695786) (width 0.2) (layer "F.Cu") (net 18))
 (segment (start 132.042 95.695786) (end 146.04475 81.693036) (width 0.2) (layer "F.Cu") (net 18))
 (segment (start 114.026184 101.001) (end 128.31747 101.001) (width 0.2) (layer "F.Cu") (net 18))
 (segment (start 146.04475 70.31975) (end 144.94375 69.21875) (width 0.2) (layer "F.Cu") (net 18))
 (segment (start 92.720314 97.511) (end 95.207498 95.023816) (width 0.2) (layer "F.Cu") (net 18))
 (segment (start 95.207498 95.023816) (end 108.049 95.023816) (width 0.2) (layer "F.Cu") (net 18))
 (segment (start 146.04475 81.693036) (end 146.04475 70.31975) (width 0.2) (layer "F.Cu") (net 18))
 (segment (start 128.31747 101.001) (end 132.042 97.27647) (width 0.2) (layer "F.Cu") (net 18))
 (segment (start 91.559686 97.511) (end 92.720314 97.511) (width 0.2) (layer "F.Cu") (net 18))
 (segment (start 84.89375 90.845064) (end 91.559686 97.511) (width 0.2) (layer "F.Cu") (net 18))
 (segment (start 80.34275 87.16775) (end 80.34275 68.29275) (width 0.2) (layer "F.Cu") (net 10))
 (segment (start 80.34275 68.29275) (end 82.46775 68.29275) (width 0.2) (layer "F.Cu") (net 10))
 (segment (start 81.39375 88.21875) (end 80.34275 87.16775) (width 0.2) (layer "F.Cu") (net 10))
 (segment (start 82.46775 68.29275) (end 84.94375 70.76875) (width 0.2) (layer "F.Cu") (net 10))
 (segment (start 83.79275 109.19275) (end 85.324 110.724) (width 0.2) (layer "F.Cu") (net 9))
 (segment (start 85.324 110.724) (end 128.75447 110.724) (width 0.2) (layer "F.Cu") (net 9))
 (segment (start 81.44375 69.01875) (end 83.79275 71.36775) (width 0.2) (layer "F.Cu") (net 9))
 (segment (start 128.75447 110.724) (end 148.44375 91.03472) (width 0.2) (layer "F.Cu") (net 9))
 (segment (start 83.79275 71.36775) (end 83.79275 109.19275) (width 0.2) (layer "F.Cu") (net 9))
 (segment (start 148.44375 91.03472) (end 148.44375 89.84375) (width 0.2) (layer "F.Cu") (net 9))
 (segment (start 92.14 58.01) (end 105.07 45.08) (width 0.2) (layer "F.Cu") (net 14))
 (segment (start 105.07 45.08) (end 107.36 45.08) (width 0.2) (layer "F.Cu") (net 14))
 (segment (start 92.14 59.991314) (end 90.739 58.590314) (width 0.2) (layer "F.Cu") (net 2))
 (segment (start 92.14 77.06) (end 92.14 59.991314) (width 0.2) (layer "F.Cu") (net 2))
 (segment (start 90.739 58.590314) (end 90.739 45.847374) (width 0.2) (layer "F.Cu") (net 2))
 (segment (start 90.739 45.847374) (end 99.126374 37.46) (width 0.2) (layer "F.Cu") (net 2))
 (segment (start 99.126374 37.46) (end 107.36 37.46) (width 0.2) (layer "F.Cu") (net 2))
 (segment (start 108.423 44.63969) (end 107.38631 43.603) (width 0.2) (layer "F.Cu") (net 4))
 (segment (start 105.008 31.578374) (end 105.269374 31.317) (width 0.2) (layer "F.Cu") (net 4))
 (segment (start 105.008 39.198374) (end 105.269374 38.937) (width 0.2) (layer "F.Cu") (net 4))
 (segment (start 105.269374 43.603) (end 105.008 43.341626) (width 0.2) (layer "F.Cu") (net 4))
 (segment (start 113.917 31.317) (end 122.6 40) (width 0.2) (layer "F.Cu") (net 4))
 (segment (start 105.269374 31.317) (end 113.917 31.317) (width 0.2) (layer "F.Cu") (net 4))
 (segment (start 105.008 35.721626) (end 105.008 31.578374) (width 0.2) (layer "F.Cu") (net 4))
 (segment (start 108.423 79.827) (end 108.423 44.63969) (width 0.2) (layer "F.Cu") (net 4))
 (segment (start 105.269374 38.937) (end 110.5999 38.937) (width 0.2) (layer "F.Cu") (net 4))
 (segment (start 105.008 43.341626) (end 105.008 39.198374) (width 0.2) (layer "F.Cu") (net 4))
 (segment (start 107.6459 35.983) (end 105.269374 35.983) (width 0.2) (layer "F.Cu") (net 4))
 (segment (start 107.38631 43.603) (end 105.269374 43.603) (width 0.2) (layer "F.Cu") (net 4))
 (segment (start 105.269374 35.983) (end 105.008 35.721626) (width 0.2) (layer "F.Cu") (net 4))
 (segment (start 92.14 96.11) (end 108.423 79.827) (width 0.2) (layer "F.Cu") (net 4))
 (segment (start 110.5999 38.937) (end 107.6459 35.983) (width 0.2) (layer "F.Cu") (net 4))
 (segment (start 111.19 46.37) (end 107.36 42.54) (width 0.2) (layer "F.Cu") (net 3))
 (segment (start 111.19 58.01) (end 111.19 46.37) (width 0.2) (layer "F.Cu") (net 3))
 (segment (start 112.591 75.659) (end 112.591 45.231) (width 0.2) (layer "F.Cu") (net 13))
 (segment (start 112.591 45.231) (end 107.36 40) (width 0.2) (layer "F.Cu") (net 13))
 (segment (start 111.19 77.06) (end 112.591 75.659) (width 0.2) (layer "F.Cu") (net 13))
 (segment (start 130.820314 97.511) (end 131.641 96.690314) (width 0.2) (layer "F.Cu") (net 12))
 (segment (start 137.991 73.939686) (end 137.170314 73.119) (width 0.2) (layer "F.Cu") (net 12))
 (segment (start 137.991 75.100314) (end 137.991 73.939686) (width 0.2) (layer "F.Cu") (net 12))
 (segment (start 137.170314 56.871) (end 137.991 56.050314) (width 0.2) (layer "F.Cu") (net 12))
 (segment (start 137.170314 90.000372) (end 137.170314 75.921) (width 0.2) (layer "F.Cu") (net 12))
 (segment (start 114.276 41.076) (end 109.8 36.6) (width 0.2) (layer "F.Cu") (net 12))
 (segment (start 111.19 96.11) (end 128.258686 96.11) (width 0.2) (layer "F.Cu") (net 12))
 (segment (start 137.991 56.050314) (end 137.991 54.210274) (width 0.2) (layer "F.Cu") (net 12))
 (segment (start 124.856726 41.076) (end 114.276 41.076) (width 0.2) (layer "F.Cu") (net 12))
 (segment (start 137.170314 73.119) (end 137.170314 56.871) (width 0.2) (layer "F.Cu") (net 12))
 (segment (start 129.659686 97.511) (end 130.820314 97.511) (width 0.2) (layer "F.Cu") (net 12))
 (segment (start 128.258686 96.11) (end 129.659686 97.511) (width 0.2) (layer "F.Cu") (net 12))
 (segment (start 131.641 96.690314) (end 131.641 95.529686) (width 0.2) (layer "F.Cu") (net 12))
 (segment (start 131.641 95.529686) (end 137.170314 90.000372) (width 0.2) (layer "F.Cu") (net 12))
 (segment (start 137.991 54.210274) (end 124.856726 41.076) (width 0.2) (layer "F.Cu") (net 12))
 (segment (start 137.170314 75.921) (end 137.991 75.100314) (width 0.2) (layer "F.Cu") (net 12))
 (via (at 109.8 36.6) (size 0.6) (drill 0.3) (layers "F.Cu" "B.Cu") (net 12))
 (segment (start 109.04 36.6) (end 107.36 34.92) (width 0.2) (layer "B.Cu") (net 12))
 (segment (start 109.8 36.6) (end 109.04 36.6) (width 0.2) (layer "B.Cu") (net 12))
 (segment (start 108.423 33.443) (end 107.36 32.38) (width 0.2) (layer "F.Cu") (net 11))
 (segment (start 108.423 36.193) (end 108.423 33.443) (width 0.2) (layer "F.Cu") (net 11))
 (segment (start 130.24 58.01) (end 108.423 36.193) (width 0.2) (layer "F.Cu") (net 11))
 (segment (start 130.24 77.06) (end 131.641 75.659) (width 0.2) (layer "F.Cu") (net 16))
 (segment (start 131.641 50.50337) (end 123.67763 42.54) (width 0.2) (layer "F.Cu") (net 16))
 (segment (start 131.641 75.659) (end 131.641 50.50337) (width 0.2) (layer "F.Cu") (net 16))
 (segment (start 123.67763 42.54) (end 122.6 42.54) (width 0.2) (layer "F.Cu") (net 16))
 (segment (start 130.24 80.049314) (end 135.189 75.100314) (width 0.2) (layer "F.Cu") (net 5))
 (segment (start 132.042 52.903314) (end 132.042 48.828374) (width 0.2) (layer "F.Cu") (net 5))
 (segment (start 135.189 62.735816) (end 136.401 61.523816) (width 0.2) (layer "F.Cu") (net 5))
 (segment (start 136.401 57.262314) (end 132.042 52.903314) (width 0.2) (layer "F.Cu") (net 5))
 (segment (start 136.401 61.523816) (end 136.401 57.262314) (width 0.2) (layer "F.Cu") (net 5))
 (segment (start 130.24 96.11) (end 130.24 80.049314) (width 0.2) (layer "F.Cu") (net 5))
 (segment (start 122.15969 41.477) (end 121.537 42.09969) (width 0.2) (layer "F.Cu") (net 5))
 (segment (start 135.189 75.100314) (end 135.189 62.735816) (width 0.2) (layer "F.Cu") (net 5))
 (segment (start 132.042 48.828374) (end 124.690626 41.477) (width 0.2) (layer "F.Cu") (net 5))
 (segment (start 121.537 44.017) (end 122.6 45.08) (width 0.2) (layer "F.Cu") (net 5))
 (segment (start 121.537 42.09969) (end 121.537 44.017) (width 0.2) (layer "F.Cu") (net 5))
 (segment (start 124.690626 41.477) (end 122.15969 41.477) (width 0.2) (layer "F.Cu") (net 5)))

